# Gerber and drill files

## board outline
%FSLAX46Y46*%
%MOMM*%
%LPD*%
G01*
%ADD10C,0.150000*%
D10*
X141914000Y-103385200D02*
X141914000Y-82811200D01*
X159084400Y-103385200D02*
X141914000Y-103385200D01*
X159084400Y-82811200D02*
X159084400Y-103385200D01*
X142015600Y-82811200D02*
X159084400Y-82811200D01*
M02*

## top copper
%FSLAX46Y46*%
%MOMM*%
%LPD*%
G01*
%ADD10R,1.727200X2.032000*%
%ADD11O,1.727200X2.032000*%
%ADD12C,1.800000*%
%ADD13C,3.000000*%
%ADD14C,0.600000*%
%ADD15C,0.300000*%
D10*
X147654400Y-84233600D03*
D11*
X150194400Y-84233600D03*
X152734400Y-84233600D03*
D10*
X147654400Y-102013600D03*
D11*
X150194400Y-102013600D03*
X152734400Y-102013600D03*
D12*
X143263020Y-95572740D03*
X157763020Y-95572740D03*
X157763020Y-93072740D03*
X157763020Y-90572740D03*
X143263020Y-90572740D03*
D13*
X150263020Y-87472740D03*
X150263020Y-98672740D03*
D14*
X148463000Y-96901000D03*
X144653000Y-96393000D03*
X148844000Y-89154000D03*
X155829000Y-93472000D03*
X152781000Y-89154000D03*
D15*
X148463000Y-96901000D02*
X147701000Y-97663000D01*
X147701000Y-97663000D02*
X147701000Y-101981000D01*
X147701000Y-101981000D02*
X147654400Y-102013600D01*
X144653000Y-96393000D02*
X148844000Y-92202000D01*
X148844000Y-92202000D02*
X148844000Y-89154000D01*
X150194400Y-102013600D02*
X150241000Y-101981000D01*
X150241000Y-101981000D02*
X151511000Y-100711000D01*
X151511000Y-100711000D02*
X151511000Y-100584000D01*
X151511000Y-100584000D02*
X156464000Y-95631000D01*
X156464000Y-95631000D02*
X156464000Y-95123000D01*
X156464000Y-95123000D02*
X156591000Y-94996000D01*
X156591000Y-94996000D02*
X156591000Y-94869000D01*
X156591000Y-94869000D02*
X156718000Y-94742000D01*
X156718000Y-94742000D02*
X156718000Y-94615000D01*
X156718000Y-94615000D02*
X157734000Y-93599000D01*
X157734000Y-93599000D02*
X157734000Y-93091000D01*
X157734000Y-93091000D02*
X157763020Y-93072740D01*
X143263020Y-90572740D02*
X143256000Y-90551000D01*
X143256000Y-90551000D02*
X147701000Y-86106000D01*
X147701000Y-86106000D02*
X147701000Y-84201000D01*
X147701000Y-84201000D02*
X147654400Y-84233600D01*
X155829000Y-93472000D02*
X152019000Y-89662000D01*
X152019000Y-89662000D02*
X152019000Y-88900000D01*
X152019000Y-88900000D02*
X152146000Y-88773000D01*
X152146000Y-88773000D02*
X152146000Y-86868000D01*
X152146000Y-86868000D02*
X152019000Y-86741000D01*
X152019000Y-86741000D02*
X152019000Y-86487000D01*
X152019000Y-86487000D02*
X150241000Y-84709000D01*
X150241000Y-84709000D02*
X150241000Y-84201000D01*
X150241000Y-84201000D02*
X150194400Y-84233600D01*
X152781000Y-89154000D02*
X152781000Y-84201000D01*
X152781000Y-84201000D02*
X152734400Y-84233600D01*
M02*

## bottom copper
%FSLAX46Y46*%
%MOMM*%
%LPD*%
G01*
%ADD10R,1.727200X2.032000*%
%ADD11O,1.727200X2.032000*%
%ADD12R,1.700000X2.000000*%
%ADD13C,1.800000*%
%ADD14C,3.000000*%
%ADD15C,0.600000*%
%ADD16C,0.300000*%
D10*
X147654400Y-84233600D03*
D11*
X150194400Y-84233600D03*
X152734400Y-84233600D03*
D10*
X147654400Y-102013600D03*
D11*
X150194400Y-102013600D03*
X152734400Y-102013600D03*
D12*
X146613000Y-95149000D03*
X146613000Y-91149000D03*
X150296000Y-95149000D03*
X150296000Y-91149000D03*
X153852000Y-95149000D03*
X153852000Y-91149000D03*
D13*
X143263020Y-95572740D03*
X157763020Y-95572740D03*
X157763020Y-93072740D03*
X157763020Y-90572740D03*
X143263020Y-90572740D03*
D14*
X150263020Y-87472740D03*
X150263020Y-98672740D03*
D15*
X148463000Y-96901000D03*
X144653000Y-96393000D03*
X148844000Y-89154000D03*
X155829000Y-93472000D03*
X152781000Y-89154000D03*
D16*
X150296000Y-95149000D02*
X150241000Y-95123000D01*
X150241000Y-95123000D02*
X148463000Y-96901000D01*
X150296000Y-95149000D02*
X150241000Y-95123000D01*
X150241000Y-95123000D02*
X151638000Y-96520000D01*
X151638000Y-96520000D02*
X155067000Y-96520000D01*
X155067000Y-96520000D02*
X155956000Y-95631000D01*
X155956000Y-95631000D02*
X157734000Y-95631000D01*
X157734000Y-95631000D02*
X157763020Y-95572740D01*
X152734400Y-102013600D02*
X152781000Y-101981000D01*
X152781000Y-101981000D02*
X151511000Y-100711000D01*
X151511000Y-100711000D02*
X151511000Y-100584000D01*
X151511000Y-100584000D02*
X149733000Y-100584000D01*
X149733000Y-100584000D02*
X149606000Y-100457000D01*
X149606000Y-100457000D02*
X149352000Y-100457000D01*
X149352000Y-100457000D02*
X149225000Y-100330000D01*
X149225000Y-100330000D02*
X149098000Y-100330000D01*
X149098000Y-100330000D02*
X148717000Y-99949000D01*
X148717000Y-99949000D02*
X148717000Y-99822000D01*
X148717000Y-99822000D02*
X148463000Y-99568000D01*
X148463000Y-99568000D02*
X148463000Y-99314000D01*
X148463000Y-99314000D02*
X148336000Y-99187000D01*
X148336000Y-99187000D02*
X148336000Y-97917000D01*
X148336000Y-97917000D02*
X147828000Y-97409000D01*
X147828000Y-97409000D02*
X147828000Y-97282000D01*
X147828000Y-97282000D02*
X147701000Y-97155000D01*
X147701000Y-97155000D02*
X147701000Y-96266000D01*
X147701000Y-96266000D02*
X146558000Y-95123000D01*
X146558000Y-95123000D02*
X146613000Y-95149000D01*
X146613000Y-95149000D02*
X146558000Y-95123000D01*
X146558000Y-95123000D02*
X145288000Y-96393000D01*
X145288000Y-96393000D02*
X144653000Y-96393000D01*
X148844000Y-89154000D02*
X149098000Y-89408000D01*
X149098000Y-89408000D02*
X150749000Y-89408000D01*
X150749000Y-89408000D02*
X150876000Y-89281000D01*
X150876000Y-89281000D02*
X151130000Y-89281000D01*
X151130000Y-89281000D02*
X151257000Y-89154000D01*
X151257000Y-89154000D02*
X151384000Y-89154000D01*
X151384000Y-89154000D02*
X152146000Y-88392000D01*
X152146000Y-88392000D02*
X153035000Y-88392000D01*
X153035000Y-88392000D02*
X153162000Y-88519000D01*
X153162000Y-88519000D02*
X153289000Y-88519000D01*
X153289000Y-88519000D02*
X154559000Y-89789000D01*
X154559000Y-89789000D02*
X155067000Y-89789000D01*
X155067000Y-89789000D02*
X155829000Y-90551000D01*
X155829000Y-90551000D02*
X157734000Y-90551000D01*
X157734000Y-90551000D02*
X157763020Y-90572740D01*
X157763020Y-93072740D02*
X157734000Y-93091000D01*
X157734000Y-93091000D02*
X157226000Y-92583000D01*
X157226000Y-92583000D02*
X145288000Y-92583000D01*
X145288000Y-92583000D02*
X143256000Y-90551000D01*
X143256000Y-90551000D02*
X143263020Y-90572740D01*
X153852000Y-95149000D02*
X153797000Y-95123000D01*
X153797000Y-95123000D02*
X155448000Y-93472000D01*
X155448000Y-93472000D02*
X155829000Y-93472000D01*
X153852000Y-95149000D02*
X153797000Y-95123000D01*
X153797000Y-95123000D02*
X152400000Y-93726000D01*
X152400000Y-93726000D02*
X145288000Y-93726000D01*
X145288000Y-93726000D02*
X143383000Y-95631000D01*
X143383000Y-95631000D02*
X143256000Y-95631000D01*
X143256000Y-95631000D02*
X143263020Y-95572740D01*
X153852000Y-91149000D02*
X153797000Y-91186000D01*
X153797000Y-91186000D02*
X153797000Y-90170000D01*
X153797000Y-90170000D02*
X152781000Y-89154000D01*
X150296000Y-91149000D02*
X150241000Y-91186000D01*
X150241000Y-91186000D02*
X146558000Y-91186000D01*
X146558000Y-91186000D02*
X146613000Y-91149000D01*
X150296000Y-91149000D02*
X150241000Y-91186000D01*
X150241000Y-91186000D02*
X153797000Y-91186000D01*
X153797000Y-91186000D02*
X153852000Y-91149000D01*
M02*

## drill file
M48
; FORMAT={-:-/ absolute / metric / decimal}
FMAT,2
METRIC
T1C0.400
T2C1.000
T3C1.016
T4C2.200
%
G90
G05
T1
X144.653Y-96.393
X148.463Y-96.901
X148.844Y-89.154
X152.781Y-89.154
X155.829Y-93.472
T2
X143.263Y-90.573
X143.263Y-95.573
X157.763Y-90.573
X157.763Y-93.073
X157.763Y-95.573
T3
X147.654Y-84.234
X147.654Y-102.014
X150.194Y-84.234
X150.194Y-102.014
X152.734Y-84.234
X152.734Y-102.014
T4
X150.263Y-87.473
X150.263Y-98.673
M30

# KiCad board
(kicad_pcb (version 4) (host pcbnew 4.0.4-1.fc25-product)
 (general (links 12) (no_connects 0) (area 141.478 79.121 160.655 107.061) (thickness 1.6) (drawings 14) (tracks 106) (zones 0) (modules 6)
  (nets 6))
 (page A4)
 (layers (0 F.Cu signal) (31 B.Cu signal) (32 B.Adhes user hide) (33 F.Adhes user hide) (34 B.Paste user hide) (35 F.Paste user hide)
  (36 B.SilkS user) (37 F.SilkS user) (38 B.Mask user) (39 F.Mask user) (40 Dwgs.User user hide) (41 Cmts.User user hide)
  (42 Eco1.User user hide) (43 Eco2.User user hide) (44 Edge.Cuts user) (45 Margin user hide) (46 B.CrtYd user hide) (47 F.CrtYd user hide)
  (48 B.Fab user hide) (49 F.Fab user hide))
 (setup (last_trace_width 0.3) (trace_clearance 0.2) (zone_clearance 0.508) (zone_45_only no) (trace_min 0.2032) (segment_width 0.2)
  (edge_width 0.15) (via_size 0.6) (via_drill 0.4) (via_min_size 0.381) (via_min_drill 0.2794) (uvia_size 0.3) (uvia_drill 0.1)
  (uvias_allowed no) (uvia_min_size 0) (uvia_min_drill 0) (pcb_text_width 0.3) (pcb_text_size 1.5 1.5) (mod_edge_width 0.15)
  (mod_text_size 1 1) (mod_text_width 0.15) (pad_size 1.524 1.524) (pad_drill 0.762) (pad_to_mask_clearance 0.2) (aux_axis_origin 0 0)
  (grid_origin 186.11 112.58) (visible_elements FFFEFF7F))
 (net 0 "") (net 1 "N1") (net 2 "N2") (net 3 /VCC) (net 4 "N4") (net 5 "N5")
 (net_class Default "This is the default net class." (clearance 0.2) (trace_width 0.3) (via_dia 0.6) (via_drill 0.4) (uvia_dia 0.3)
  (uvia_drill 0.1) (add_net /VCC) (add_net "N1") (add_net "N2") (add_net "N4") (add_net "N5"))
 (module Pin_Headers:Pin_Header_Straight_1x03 (layer F.Cu) (at 147.6544 84.2336 90)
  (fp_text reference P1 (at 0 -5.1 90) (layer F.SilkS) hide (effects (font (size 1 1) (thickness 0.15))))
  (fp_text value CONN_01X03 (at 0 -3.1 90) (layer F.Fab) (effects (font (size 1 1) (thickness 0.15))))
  (pad 1 thru_hole rect (at 0 0 90) (size 2.032 1.7272) (drill 1.016) (layers *.Cu *.Mask F.SilkS) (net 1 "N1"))
  (pad 2 thru_hole oval (at 0 2.54 90) (size 2.032 1.7272) (drill 1.016) (layers *.Cu *.Mask F.SilkS) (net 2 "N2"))
  (pad 3 thru_hole oval (at 0 5.08 90) (size 2.032 1.7272) (drill 1.016) (layers *.Cu *.Mask F.SilkS) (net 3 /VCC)))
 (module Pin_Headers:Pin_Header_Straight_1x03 (layer F.Cu) (at 147.6544 102.0136 90)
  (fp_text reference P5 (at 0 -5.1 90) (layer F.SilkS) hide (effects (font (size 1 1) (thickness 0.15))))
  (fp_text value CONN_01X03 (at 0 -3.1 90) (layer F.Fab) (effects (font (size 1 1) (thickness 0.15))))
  (pad 1 thru_hole rect (at 0 0 90) (size 2.032 1.7272) (drill 1.016) (layers *.Cu *.Mask F.SilkS) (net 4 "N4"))
  (pad 2 thru_hole oval (at 0 2.54 90) (size 2.032 1.7272) (drill 1.016) (layers *.Cu *.Mask F.SilkS) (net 1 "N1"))
  (pad 3 thru_hole oval (at 0 5.08 90) (size 2.032 1.7272) (drill 1.016) (layers *.Cu *.Mask F.SilkS) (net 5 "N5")))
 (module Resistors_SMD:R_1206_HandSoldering (layer B.Cu) (at 146.613 93.149 90)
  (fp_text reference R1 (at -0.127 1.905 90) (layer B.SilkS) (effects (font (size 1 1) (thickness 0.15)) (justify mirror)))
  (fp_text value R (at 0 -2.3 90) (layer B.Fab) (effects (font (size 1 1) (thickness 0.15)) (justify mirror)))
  (pad 1 smd rect (at -2 0 90) (size 2 1.7) (layers B.Cu B.Paste B.Mask) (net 5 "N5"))
  (pad 2 smd rect (at 2 0 90) (size 2 1.7) (layers B.Cu B.Paste B.Mask) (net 3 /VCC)))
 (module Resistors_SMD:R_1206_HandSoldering (layer B.Cu) (at 150.296 93.149 90)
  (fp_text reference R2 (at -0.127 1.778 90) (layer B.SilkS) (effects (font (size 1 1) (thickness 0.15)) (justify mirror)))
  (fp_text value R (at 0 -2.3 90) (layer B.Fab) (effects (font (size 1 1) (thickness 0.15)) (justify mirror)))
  (pad 1 smd rect (at -2 0 90) (size 2 1.7) (layers B.Cu B.Paste B.Mask) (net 4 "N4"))
  (pad 2 smd rect (at 2 0 90) (size 2 1.7) (layers B.Cu B.Paste B.Mask) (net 3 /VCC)))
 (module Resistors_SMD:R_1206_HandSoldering (layer B.Cu) (at 153.852 93.149 90)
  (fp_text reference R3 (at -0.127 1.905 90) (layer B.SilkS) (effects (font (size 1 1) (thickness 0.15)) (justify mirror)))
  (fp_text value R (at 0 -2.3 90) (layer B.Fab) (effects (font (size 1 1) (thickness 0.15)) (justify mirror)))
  (pad 1 smd rect (at -2 0 90) (size 2 1.7) (layers B.Cu B.Paste B.Mask) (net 2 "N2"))
  (pad 2 smd rect (at 2 0 90) (size 2 1.7) (layers B.Cu B.Paste B.Mask) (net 3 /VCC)))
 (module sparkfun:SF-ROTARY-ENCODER (layer F.Cu) (at 150.26302 93.07274 90)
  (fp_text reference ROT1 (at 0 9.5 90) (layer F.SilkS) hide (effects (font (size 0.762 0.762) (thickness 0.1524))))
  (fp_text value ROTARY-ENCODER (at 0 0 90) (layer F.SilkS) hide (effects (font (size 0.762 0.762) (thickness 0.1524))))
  (pad 1 thru_hole circle (at -2.5 -7 90) (size 1.8 1.8) (drill 1) (layers *.Cu *.Mask F.SilkS) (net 2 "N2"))
  (pad 2 thru_hole circle (at -2.5 7.5 90) (size 1.8 1.8) (drill 1) (layers *.Cu *.Mask F.SilkS) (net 4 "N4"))
  (pad 3 thru_hole circle (at 0 7.5 90) (size 1.8 1.8) (drill 1) (layers *.Cu *.Mask F.SilkS) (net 1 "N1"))
  (pad 4 thru_hole circle (at 2.5 7.5 90) (size 1.8 1.8) (drill 1) (layers *.Cu *.Mask F.SilkS) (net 5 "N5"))
  (pad 5 thru_hole circle (at 2.5 -7 90) (size 1.8 1.8) (drill 1) (layers *.Cu *.Mask F.SilkS) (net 1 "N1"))
  (pad "" thru_hole circle (at 5.6 0 90) (size 3 3) (drill 2.2) (layers *.Cu *.Mask F.SilkS))
  (pad "" thru_hole circle (at -5.6 0 90) (size 3 3) (drill 2.2) (layers *.Cu *.Mask F.SilkS)))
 (gr_line (start 141.914 103.3852) (end 141.914 82.8112) (angle 90) (layer Edge.Cuts) (width 0.15))
 (gr_line (start 159.0844 103.3852) (end 141.914 103.3852) (angle 90) (layer Edge.Cuts) (width 0.15))
 (gr_line (start 159.0844 82.8112) (end 159.0844 103.3852) (angle 90) (layer Edge.Cuts) (width 0.15))
 (gr_line (start 142.0156 82.8112) (end 159.0844 82.8112) (angle 90) (layer Edge.Cuts) (width 0.15))
 (segment (start 150.296 95.149) (end 150.241 95.123) (width 0.3) (layer B.Cu) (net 4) (status 80000))
 (segment (start 150.241 95.123) (end 148.463 96.901) (width 0.3) (layer B.Cu) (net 4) (status 80000))
 (segment (start 148.463 96.901) (end 147.701 97.663) (width 0.3) (layer F.Cu) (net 4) (status 80000))
 (segment (start 147.701 97.663) (end 147.701 101.981) (width 0.3) (layer F.Cu) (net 4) (status 80000))
 (segment (start 147.701 101.981) (end 147.6544 102.0136) (width 0.3) (layer F.Cu) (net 4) (status 80000))
 (segment (start 150.296 95.149) (end 150.241 95.123) (width 0.3) (layer B.Cu) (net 4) (status 80000))
 (segment (start 150.241 95.123) (end 151.638 96.52) (width 0.3) (layer B.Cu) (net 4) (status 80000))
 (segment (start 151.638 96.52) (end 155.067 96.52) (width 0.3) (layer B.Cu) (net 4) (status 80000))
 (segment (start 155.067 96.52) (end 155.956 95.631) (width 0.3) (layer B.Cu) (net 4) (status 80000))
 (segment (start 155.956 95.631) (end 157.734 95.631) (width 0.3) (layer B.Cu) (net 4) (status 80000))
 (segment (start 157.734 95.631) (end 157.76302 95.57274) (width 0.3) (layer B.Cu) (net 4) (status 80000))
 (segment (start 152.7344 102.0136) (end 152.781 101.981) (width 0.3) (layer B.Cu) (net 5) (status 80000))
 (segment (start 152.781 101.981) (end 151.511 100.711) (width 0.3) (layer B.Cu) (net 5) (status 80000))
 (segment (start 151.511 100.711) (end 151.511 100.584) (width 0.3) (layer B.Cu) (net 5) (status 80000))
 (segment (start 151.511 100.584) (end 149.733 100.584) (width 0.3) (layer B.Cu) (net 5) (status 80000))
 (segment (start 149.733 100.584) (end 149.606 100.457) (width 0.3) (layer B.Cu) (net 5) (status 80000))
 (segment (start 149.606 100.457) (end 149.352 100.457) (width 0.3) (layer B.Cu) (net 5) (status 80000))
 (segment (start 149.352 100.457) (end 149.225 100.33) (width 0.3) (layer B.Cu) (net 5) (status 80000))
 (segment (start 149.225 100.33) (end 149.098 100.33) (width 0.3) (layer B.Cu) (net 5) (status 80000))
 (segment (start 149.098 100.33) (end 148.717 99.949) (width 0.3) (layer B.Cu) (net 5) (status 80000))
 (segment (start 148.717 99.949) (end 148.717 99.822) (width 0.3) (layer B.Cu) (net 5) (status 80000))
 (segment (start 148.717 99.822) (end 148.463 99.568) (width 0.3) (layer B.Cu) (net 5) (status 80000))
 (segment (start 148.463 99.568) (end 148.463 99.314) (width 0.3) (layer B.Cu) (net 5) (status 80000))
 (segment (start 148.463 99.314) (end 148.336 99.187) (width 0.3) (layer B.Cu) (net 5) (status 80000))
 (segment (start 148.336 99.187) (end 148.336 97.917) (width 0.3) (layer B.Cu) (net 5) (status 80000))
 (segment (start 148.336 97.917) (end 147.828 97.409) (width 0.3) (layer B.Cu) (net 5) (status 80000))
 (segment (start 147.828 97.409) (end 147.828 97.282) (width 0.3) (layer B.Cu) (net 5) (status 80000))
 (segment (start 147.828 97.282) (end 147.701 97.155) (width 0.3) (layer B.Cu) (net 5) (status 80000))
 (segment (start 147.701 97.155) (end 147.701 96.266) (width 0.3) (layer B.Cu) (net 5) (status 80000))
 (segment (start 147.701 96.266) (end 146.558 95.123) (width 0.3) (layer B.Cu) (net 5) (status 80000))
 (segment (start 146.558 95.123) (end 146.613 95.149) (width 0.3) (layer B.Cu) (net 5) (status 80000))
 (segment (start 146.613 95.149) (end 146.558 95.123) (width 0.3) (layer B.Cu) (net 5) (status 80000))
 (segment (start 146.558 95.123) (end 145.288 96.393) (width 0.3) (layer B.Cu) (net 5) (status 80000))
 (segment (start 145.288 96.393) (end 144.653 96.393) (width 0.3) (layer B.Cu) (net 5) (status 80000))
 (segment (start 144.653 96.393) (end 148.844 92.202) (width 0.3) (layer F.Cu) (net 5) (status 80000))
 (segment (start 148.844 92.202) (end 148.844 89.154) (width 0.3) (layer F.Cu) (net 5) (status 80000))
 (segment (start 148.844 89.154) (end 149.098 89.408) (width 0.3) (layer B.Cu) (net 5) (status 80000))
 (segment (start 149.098 89.408) (end 150.749 89.408) (width 0.3) (layer B.Cu) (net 5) (status 80000))
 (segment (start 150.749 89.408) (end 150.876 89.281) (width 0.3) (layer B.Cu) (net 5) (status 80000))
 (segment (start 150.876 89.281) (end 151.13 89.281) (width 0.3) (layer B.Cu) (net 5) (status 80000))
 (segment (start 151.13 89.281) (end 151.257 89.154) (width 0.3) (layer B.Cu) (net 5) (status 80000))
 (segment (start 151.257 89.154) (end 151.384 89.154) (width 0.3) (layer B.Cu) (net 5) (status 80000))
 (segment (start 151.384 89.154) (end 152.146 88.392) (width 0.3) (layer B.Cu) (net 5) (status 80000))
 (segment (start 152.146 88.392) (end 153.035 88.392) (width 0.3) (layer B.Cu) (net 5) (status 80000))
 (segment (start 153.035 88.392) (end 153.162 88.519) (width 0.3) (layer B.Cu) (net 5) (status 80000))
 (segment (start 153.162 88.519) (end 153.289 88.519) (width 0.3) (layer B.Cu) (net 5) (status 80000))
 (segment (start 153.289 88.519) (end 154.559 89.789) (width 0.3) (layer B.Cu) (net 5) (status 80000))
 (segment (start 154.559 89.789) (end 155.067 89.789) (width 0.3) (layer B.Cu) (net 5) (status 80000))
 (segment (start 155.067 89.789) (end 155.829 90.551) (width 0.3) (layer B.Cu) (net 5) (status 80000))
 (segment (start 155.829 90.551) (end 157.734 90.551) (width 0.3) (layer B.Cu) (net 5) (status 80000))
 (segment (start 157.734 90.551) (end 157.76302 90.57274) (width 0.3) (layer B.Cu) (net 5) (status 80000))
 (segment (start 150.1944 102.0136) (end 150.241 101.981) (width 0.3) (layer F.Cu) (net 1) (status 80000))
 (segment (start 150.241 101.981) (end 151.511 100.711) (width 0.3) (layer F.Cu) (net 1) (status 80000))
 (segment (start 151.511 100.711) (end 151.511 100.584) (width 0.3) (layer F.Cu) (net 1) (status 80000))
 (segment (start 151.511 100.584) (end 156.464 95.631) (width 0.3) (layer F.Cu) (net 1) (status 80000))
 (segment (start 156.464 95.631) (end 156.464 95.123) (width 0.3) (layer F.Cu) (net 1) (status 80000))
 (segment (start 156.464 95.123) (end 156.591 94.996) (width 0.3) (layer F.Cu) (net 1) (status 80000))
 (segment (start 156.591 94.996) (end 156.591 94.869) (width 0.3) (layer F.Cu) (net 1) (status 80000))
 (segment (start 156.591 94.869) (end 156.718 94.742) (width 0.3) (layer F.Cu) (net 1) (status 80000))
 (segment (start 156.718 94.742) (end 156.718 94.615) (width 0.3) (layer F.Cu) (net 1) (status 80000))
 (segment (start 156.718 94.615) (end 157.734 93.599) (width 0.3) (layer F.Cu) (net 1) (status 80000))
 (segment (start 157.734 93.599) (end 157.734 93.091) (width 0.3) (layer F.Cu) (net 1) (status 80000))
 (segment (start 157.734 93.091) (end 157.76302 93.07274) (width 0.3) (layer F.Cu) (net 1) (status 80000))
 (segment (start 143.26302 90.57274) (end 143.256 90.551) (width 0.3) (layer F.Cu) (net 1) (status 80000))
 (segment (start 143.256 90.551) (end 147.701 86.106) (width 0.3) (layer F.Cu) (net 1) (status 80000))
 (segment (start 147.701 86.106) (end 147.701 84.201) (width 0.3) (layer F.Cu) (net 1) (status 80000))
 (segment (start 147.701 84.201) (end 147.6544 84.2336) (width 0.3) (layer F.Cu) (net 1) (status 80000))
 (segment (start 157.76302 93.07274) (end 157.734 93.091) (width 0.3) (layer B.Cu) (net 1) (status 80000))
 (segment (start 157.734 93.091) (end 157.226 92.583) (width 0.3) (layer B.Cu) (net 1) (status 80000))
 (segment (start 157.226 92.583) (end 145.288 92.583) (width 0.3) (layer B.Cu) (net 1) (status 80000))
 (segment (start 145.288 92.583) (end 143.256 90.551) (width 0.3) (layer B.Cu) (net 1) (status 80000))
 (segment (start 143.256 90.551) (end 143.26302 90.57274) (width 0.3) (layer B.Cu) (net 1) (status 80000))
 (segment (start 153.852 95.149) (end 153.797 95.123) (width 0.3) (layer B.Cu) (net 2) (status 80000))
 (segment (start 153.797 95.123) (end 155.448 93.472) (width 0.3) (layer B.Cu) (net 2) (status 80000))
 (segment (start 155.448 93.472) (end 155.829 93.472) (width 0.3) (layer B.Cu) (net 2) (status 80000))
 (segment (start 155.829 93.472) (end 152.019 89.662) (width 0.3) (layer F.Cu) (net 2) (status 80000))
 (segment (start 152.019 89.662) (end 152.019 88.9) (width 0.3) (layer F.Cu) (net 2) (status 80000))
 (segment (start 152.019 88.9) (end 152.146 88.773) (width 0.3) (layer F.Cu) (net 2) (status 80000))
 (segment (start 152.146 88.773) (end 152.146 86.868) (width 0.3) (layer F.Cu) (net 2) (status 80000))
 (segment (start 152.146 86.868) (end 152.019 86.741) (width 0.3) (layer F.Cu) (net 2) (status 80000))
 (segment (start 152.019 86.741) (end 152.019 86.487) (width 0.3) (layer F.Cu) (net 2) (status 80000))
 (segment (start 152.019 86.487) (end 150.241 84.709) (width 0.3) (layer F.Cu) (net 2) (status 80000))
 (segment (start 150.241 84.709) (end 150.241 84.201) (width 0.3) (layer F.Cu) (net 2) (status 80000))
 (segment (start 150.241 84.201) (end 150.1944 84.2336) (width 0.3) (layer F.Cu) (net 2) (status 80000))
 (segment (start 153.852 95.149) (end 153.797 95.123) (width 0.3) (layer B.Cu) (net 2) (status 80000))
 (segment (start 153.797 95.123) (end 152.4 93.726) (width 0.3) (layer B.Cu) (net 2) (status 80000))
 (segment (start 152.4 93.726) (end 145.288 93.726) (width 0.3) (layer B.Cu) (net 2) (status 80000))
 (segment (start 145.288 93.726) (end 143.383 95.631) (width 0.3) (layer B.Cu) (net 2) (status 80000))
 (segment (start 143.383 95.631) (end 143.256 95.631) (width 0.3) (layer B.Cu) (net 2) (status 80000))
 (segment (start 143.256 95.631) (end 143.26302 95.57274) (width 0.3) (layer B.Cu) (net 2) (status 80000))
 (segment (start 153.852 91.149) (end 153.797 91.186) (width 0.3) (layer B.Cu) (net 3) (status 80000))
 (segment (start 153.797 91.186) (end 153.797 90.17) (width 0.3) (layer B.Cu) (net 3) (status 80000))
 (segment (start 153.797 90.17) (end 152.781 89.154) (width 0.3) (layer B.Cu) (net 3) (status 80000))
 (segment (start 152.781 89.154) (end 152.781 84.201) (width 0.3) (layer F.Cu) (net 3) (status 80000))
 (segment (start 152.781 84.201) (end 152.7344 84.2336) (width 0.3) (layer F.Cu) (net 3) (status 80000))
 (segment (start 150.296 91.149) (end 150.241 91.186) (width 0.3) (layer B.Cu) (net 3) (status 80000))
 (segment (start 150.241 91.186) (end 146.558 91.186) (width 0.3) (layer B.Cu) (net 3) (status 80000))
 (segment (start 146.558 91.186) (end 146.613 91.149) (width 0.3) (layer B.Cu) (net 3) (status 80000))
 (segment (start 150.296 91.149) (end 150.241 91.186) (width 0.3) (layer B.Cu) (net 3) (status 80000))
 (segment (start 150.241 91.186) (end 153.797 91.186) (width 0.3) (layer B.Cu) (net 3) (status 80000))
 (segment (start 153.797 91.186) (end 153.852 91.149) (width 0.3) (layer B.Cu) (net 3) (status 80000))
 (via (at 148.463 96.901) (size 0.6) (layers F.Cu B.Cu) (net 4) (status 80000))
 (via (at 144.653 96.393) (size 0.6) (layers F.Cu B.Cu) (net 5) (status 80000))
 (via (at 148.844 89.154) (size 0.6) (layers F.Cu B.Cu) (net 5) (status 80000))
 (via (at 155.829 93.472) (size 0.6) (layers F.Cu B.Cu) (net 2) (status 80000))
 (via (at 152.781 89.154) (size 0.6) (layers F.Cu B.Cu) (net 3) (status 80000)))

